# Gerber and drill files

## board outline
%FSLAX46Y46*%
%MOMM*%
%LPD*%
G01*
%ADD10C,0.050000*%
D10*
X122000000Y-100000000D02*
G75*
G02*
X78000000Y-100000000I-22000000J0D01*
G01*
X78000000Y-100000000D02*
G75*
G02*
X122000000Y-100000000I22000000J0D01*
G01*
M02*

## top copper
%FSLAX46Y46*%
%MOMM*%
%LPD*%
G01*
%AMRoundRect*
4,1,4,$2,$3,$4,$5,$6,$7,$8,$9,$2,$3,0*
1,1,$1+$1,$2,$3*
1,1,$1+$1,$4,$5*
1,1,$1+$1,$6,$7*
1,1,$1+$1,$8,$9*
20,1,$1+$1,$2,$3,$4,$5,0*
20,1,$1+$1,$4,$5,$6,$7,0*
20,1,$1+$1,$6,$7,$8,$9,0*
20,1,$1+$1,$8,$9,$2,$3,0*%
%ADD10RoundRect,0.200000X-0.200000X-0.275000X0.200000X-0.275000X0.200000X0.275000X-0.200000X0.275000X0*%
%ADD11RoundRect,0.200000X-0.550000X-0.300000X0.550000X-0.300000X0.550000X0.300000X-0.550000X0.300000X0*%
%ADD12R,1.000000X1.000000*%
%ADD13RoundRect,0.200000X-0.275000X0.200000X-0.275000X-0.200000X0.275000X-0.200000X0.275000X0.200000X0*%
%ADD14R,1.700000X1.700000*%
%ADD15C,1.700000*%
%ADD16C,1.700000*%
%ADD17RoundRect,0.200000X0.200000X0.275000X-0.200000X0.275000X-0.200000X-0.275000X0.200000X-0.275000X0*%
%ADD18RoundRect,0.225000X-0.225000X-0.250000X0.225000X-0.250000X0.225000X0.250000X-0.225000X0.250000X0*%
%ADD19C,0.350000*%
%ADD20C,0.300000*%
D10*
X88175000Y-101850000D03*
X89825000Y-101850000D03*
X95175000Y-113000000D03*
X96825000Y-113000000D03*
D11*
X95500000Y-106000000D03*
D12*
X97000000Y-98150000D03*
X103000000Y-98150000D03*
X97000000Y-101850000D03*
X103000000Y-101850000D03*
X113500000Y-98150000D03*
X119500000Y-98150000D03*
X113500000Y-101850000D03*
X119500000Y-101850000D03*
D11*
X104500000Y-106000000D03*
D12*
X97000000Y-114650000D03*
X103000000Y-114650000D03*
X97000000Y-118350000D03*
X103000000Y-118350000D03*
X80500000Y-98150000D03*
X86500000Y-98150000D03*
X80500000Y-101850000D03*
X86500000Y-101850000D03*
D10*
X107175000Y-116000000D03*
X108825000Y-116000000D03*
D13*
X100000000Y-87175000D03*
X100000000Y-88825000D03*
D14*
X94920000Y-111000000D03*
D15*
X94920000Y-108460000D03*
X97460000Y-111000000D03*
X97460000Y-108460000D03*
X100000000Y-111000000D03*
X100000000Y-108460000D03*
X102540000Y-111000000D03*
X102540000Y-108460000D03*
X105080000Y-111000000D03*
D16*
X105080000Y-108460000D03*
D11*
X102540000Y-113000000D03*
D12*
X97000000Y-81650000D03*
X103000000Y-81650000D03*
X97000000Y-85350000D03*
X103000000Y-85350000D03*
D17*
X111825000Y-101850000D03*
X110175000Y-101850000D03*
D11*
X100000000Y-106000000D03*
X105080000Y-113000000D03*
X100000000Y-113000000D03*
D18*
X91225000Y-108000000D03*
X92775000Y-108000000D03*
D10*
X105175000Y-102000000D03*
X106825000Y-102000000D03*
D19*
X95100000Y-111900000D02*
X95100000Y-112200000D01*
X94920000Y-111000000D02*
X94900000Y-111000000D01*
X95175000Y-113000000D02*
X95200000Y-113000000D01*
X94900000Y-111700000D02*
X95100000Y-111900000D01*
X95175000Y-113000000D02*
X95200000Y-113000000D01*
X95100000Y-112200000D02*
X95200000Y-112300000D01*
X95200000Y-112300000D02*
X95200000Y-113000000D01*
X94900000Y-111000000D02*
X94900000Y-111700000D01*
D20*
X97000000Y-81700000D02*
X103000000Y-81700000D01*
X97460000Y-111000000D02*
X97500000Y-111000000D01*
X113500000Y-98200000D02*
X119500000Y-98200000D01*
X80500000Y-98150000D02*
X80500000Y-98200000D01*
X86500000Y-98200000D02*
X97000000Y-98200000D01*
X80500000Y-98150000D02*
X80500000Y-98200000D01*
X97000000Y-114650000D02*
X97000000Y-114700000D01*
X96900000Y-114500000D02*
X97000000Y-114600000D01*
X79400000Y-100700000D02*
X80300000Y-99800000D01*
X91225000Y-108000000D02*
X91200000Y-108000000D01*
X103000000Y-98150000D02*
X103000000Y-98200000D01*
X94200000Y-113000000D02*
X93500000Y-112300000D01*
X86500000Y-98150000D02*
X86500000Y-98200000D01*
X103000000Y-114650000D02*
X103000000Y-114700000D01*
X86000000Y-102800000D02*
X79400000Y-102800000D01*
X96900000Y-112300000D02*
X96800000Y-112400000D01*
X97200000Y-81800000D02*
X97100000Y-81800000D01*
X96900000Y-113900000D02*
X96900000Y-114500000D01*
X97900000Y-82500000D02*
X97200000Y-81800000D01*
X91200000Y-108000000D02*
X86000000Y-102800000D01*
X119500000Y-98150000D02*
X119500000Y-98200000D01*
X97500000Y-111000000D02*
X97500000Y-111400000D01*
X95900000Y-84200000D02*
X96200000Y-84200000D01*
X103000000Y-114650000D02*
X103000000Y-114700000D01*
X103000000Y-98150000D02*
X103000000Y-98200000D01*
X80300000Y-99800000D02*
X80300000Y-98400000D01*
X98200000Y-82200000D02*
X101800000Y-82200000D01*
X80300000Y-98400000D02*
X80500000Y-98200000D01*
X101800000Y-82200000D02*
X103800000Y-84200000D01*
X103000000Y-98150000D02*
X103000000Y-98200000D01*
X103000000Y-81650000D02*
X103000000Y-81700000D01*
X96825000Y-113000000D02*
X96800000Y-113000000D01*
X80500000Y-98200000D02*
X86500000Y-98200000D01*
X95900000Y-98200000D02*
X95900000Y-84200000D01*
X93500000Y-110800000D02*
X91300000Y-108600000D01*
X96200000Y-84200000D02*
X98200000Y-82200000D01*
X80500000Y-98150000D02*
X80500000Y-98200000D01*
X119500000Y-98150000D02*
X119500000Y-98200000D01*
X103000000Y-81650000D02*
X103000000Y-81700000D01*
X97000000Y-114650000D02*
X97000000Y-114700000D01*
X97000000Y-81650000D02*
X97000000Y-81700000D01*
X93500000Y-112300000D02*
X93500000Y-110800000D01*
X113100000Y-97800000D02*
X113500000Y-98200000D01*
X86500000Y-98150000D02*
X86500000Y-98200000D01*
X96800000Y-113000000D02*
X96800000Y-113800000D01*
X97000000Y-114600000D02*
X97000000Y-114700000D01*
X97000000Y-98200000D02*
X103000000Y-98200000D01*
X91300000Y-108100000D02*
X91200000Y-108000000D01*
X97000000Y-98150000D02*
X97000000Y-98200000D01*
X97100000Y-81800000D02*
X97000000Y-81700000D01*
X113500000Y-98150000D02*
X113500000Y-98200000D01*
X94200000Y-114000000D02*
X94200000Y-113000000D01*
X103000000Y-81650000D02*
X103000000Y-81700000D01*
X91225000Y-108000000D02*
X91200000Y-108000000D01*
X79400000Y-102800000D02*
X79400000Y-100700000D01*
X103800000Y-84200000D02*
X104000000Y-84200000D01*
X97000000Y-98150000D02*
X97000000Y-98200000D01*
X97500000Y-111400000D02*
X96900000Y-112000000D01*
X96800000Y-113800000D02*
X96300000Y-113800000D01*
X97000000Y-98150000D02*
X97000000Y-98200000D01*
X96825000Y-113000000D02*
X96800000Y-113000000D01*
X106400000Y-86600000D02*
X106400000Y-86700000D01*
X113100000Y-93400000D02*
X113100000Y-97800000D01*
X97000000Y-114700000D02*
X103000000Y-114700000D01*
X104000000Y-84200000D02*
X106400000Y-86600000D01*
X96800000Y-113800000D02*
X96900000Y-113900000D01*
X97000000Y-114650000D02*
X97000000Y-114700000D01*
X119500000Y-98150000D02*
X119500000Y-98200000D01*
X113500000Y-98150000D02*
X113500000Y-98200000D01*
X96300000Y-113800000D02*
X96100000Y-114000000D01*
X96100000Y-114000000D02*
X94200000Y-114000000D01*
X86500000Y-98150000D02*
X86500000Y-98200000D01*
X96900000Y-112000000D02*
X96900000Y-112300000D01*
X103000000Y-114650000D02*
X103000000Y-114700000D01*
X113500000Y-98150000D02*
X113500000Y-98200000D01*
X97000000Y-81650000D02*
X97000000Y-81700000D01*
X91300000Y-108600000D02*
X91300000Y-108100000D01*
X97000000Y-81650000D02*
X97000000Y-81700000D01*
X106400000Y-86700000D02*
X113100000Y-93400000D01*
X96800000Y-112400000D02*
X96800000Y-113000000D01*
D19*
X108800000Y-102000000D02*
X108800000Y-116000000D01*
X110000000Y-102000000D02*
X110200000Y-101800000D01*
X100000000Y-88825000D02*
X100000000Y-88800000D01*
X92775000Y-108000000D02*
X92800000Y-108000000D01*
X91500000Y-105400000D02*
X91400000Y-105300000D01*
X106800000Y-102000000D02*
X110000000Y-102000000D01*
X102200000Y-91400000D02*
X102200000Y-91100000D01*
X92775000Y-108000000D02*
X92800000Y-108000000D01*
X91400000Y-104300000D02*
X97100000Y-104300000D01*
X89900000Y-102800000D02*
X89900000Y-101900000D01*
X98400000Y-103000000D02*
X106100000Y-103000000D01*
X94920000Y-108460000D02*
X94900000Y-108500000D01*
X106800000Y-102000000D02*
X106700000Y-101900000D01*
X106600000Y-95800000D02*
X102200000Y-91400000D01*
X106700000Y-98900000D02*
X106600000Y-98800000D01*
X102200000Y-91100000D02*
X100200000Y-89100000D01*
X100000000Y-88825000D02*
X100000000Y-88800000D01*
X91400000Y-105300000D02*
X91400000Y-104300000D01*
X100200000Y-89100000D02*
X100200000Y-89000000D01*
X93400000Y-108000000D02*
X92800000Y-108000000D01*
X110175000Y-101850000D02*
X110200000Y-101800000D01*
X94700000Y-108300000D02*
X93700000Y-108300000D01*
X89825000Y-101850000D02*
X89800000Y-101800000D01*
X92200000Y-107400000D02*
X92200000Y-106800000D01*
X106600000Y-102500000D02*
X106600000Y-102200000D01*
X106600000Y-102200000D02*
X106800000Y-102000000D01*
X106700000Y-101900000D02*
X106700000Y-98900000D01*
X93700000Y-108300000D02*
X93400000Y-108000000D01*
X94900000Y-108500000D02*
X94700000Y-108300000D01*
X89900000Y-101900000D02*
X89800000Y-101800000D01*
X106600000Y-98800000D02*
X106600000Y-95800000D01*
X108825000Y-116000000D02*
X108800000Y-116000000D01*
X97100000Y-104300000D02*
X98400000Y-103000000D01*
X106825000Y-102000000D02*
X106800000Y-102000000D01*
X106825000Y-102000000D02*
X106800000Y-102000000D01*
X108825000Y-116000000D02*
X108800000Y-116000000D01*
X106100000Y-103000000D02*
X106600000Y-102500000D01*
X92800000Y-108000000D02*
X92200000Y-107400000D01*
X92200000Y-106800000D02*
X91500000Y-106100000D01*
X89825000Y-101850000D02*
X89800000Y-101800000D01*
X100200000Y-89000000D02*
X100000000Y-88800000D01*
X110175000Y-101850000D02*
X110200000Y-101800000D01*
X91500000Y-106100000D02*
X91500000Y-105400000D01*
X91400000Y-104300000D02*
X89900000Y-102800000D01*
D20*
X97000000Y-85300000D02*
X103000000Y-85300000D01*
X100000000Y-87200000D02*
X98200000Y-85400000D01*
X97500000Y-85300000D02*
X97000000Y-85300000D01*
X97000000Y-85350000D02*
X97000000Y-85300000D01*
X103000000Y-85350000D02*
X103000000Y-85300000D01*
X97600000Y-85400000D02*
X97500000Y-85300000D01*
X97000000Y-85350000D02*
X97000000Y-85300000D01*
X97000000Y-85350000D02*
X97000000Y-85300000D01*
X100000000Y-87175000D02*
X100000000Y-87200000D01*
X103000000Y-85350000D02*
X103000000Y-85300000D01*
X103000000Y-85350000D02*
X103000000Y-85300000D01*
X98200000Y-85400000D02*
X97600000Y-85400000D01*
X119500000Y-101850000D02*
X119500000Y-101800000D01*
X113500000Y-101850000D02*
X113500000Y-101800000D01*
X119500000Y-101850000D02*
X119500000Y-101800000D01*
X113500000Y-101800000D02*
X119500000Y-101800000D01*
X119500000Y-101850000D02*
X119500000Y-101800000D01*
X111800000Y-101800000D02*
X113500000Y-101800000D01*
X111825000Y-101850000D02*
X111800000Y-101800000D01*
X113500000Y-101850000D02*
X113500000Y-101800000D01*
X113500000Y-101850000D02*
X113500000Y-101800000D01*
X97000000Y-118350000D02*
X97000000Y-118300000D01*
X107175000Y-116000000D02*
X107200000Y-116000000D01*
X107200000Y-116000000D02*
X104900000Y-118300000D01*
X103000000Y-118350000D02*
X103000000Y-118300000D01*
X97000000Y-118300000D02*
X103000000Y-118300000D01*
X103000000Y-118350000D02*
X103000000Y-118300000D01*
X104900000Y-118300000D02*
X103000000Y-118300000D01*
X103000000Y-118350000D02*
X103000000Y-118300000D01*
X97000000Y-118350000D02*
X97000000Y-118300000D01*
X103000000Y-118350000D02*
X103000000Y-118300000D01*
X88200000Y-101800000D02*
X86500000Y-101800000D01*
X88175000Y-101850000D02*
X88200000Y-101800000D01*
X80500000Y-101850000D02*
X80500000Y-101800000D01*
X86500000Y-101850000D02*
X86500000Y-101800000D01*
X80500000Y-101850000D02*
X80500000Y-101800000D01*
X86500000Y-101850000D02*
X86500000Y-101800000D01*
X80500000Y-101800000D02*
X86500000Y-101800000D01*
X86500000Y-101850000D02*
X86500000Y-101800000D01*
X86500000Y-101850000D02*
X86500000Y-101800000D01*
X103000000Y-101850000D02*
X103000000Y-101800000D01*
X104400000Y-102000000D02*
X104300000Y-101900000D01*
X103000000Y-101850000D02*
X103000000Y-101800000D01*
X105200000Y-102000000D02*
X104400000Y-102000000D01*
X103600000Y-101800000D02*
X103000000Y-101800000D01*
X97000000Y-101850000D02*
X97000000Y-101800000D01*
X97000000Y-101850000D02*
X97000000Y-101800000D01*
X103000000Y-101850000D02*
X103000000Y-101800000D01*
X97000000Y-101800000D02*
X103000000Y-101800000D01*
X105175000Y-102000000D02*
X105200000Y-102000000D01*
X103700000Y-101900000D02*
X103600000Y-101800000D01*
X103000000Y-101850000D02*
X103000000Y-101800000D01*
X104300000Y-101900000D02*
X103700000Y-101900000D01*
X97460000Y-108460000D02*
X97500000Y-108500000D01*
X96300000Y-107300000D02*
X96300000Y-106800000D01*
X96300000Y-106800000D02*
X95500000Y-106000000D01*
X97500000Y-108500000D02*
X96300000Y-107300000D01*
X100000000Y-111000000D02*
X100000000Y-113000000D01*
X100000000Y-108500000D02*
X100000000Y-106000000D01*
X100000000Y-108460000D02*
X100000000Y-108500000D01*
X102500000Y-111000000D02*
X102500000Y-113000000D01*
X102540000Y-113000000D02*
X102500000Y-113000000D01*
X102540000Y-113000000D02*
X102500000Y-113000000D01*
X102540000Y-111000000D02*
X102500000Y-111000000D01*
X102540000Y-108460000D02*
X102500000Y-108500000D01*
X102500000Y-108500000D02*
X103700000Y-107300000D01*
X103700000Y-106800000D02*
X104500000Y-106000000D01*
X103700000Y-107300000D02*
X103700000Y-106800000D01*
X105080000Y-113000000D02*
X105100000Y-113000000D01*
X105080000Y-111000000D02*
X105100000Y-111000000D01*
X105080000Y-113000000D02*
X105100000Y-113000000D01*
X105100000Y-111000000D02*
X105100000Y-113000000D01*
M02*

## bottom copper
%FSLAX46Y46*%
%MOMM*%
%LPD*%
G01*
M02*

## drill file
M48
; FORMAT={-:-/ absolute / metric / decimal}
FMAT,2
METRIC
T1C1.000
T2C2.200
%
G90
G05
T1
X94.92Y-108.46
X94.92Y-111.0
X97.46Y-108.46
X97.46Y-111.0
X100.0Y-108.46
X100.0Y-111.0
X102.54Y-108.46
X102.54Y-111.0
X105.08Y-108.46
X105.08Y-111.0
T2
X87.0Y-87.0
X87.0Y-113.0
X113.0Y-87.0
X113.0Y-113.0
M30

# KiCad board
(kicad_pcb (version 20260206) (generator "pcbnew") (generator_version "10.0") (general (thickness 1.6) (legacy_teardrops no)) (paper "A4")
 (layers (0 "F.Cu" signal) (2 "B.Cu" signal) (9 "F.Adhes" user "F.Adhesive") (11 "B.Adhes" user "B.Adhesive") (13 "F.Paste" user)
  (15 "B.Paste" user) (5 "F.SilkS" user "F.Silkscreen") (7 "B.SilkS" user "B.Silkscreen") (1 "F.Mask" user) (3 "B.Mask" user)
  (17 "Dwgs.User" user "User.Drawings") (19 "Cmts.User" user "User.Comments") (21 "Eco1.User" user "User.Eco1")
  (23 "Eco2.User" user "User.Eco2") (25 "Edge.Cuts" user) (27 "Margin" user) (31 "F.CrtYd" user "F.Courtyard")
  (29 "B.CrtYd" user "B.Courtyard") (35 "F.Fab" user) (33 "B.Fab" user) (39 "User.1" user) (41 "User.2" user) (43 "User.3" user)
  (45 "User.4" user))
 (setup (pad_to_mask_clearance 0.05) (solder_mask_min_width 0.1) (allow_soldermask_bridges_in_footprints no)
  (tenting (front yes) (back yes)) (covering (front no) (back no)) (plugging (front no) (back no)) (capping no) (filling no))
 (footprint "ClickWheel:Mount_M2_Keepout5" (layer "F.Cu") (at 87 113)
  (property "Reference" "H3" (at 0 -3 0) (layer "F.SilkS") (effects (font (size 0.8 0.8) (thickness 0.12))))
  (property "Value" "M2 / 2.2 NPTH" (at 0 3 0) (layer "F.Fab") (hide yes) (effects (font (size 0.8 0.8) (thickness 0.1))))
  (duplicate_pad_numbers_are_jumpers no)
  (pad "" np_thru_hole circle (at 0 0) (size 2.2 2.2) (drill 2.2) (layers "*.Cu" "*.Mask")))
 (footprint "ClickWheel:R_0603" (layer "F.Cu") (at 89 101.85)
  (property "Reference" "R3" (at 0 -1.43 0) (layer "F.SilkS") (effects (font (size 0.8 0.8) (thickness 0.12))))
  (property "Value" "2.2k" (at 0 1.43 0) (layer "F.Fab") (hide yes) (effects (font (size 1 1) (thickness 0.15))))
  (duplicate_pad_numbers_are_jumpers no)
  (pad "1" smd roundrect (at -0.825 0) (size 0.8 0.95) (layers "F.Cu" "F.Mask" "F.Paste") (roundrect_rratio 0.25) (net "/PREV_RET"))
  (pad "2" smd roundrect (at 0.825 0) (size 0.8 0.95) (layers "F.Cu" "F.Mask" "F.Paste") (roundrect_rratio 0.25) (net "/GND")))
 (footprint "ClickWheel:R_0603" (layer "F.Cu") (at 96 113)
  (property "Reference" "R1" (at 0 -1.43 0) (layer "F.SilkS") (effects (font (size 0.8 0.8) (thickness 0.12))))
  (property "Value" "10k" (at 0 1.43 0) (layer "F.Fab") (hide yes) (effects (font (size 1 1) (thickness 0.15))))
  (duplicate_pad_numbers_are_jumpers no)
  (pad "1" smd roundrect (at -0.825 0) (size 0.8 0.95) (layers "F.Cu" "F.Mask" "F.Paste") (roundrect_rratio 0.25) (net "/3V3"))
  (pad "2" smd roundrect (at 0.825 0) (size 0.8 0.95) (layers "F.Cu" "F.Mask" "F.Paste") (roundrect_rratio 0.25) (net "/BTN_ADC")))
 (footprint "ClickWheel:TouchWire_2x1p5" (layer "F.Cu") (at 95.5 106)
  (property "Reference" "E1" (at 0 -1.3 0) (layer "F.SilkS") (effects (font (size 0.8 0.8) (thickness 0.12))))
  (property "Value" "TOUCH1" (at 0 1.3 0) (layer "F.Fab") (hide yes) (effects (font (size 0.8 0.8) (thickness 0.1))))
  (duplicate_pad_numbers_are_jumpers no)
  (pad "1" smd roundrect (at 0 0) (size 1.5 1) (layers "F.Cu" "F.Mask") (roundrect_rratio 0.2) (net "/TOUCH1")))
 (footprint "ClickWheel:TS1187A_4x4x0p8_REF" (layer "F.Cu") (at 100 100)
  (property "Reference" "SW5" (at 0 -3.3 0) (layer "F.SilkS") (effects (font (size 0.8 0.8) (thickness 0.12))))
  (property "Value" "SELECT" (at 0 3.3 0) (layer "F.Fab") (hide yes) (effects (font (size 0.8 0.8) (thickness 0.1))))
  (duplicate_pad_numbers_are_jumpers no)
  (pad "1" smd rect (at -3 -1.85) (size 1 1) (layers "F.Cu" "F.Mask" "F.Paste") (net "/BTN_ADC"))
  (pad "1" smd rect (at 3 -1.85) (size 1 1) (layers "F.Cu" "F.Mask" "F.Paste") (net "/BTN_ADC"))
  (pad "2" smd rect (at -3 1.85) (size 1 1) (layers "F.Cu" "F.Mask" "F.Paste") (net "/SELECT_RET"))
  (pad "2" smd rect (at 3 1.85) (size 1 1) (layers "F.Cu" "F.Mask" "F.Paste") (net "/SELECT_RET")))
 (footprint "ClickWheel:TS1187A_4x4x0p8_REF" (layer "F.Cu") (at 116.5 100)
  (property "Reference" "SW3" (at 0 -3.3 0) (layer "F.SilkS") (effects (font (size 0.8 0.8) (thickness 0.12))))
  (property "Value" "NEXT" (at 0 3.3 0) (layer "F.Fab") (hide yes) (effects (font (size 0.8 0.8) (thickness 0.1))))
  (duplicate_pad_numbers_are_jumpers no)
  (pad "1" smd rect (at -3 -1.85) (size 1 1) (layers "F.Cu" "F.Mask" "F.Paste") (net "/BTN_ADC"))
  (pad "1" smd rect (at 3 -1.85) (size 1 1) (layers "F.Cu" "F.Mask" "F.Paste") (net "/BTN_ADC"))
  (pad "2" smd rect (at -3 1.85) (size 1 1) (layers "F.Cu" "F.Mask" "F.Paste") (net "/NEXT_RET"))
  (pad "2" smd rect (at 3 1.85) (size 1 1) (layers "F.Cu" "F.Mask" "F.Paste") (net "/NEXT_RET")))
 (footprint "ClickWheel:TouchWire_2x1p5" (layer "F.Cu") (at 104.5 106)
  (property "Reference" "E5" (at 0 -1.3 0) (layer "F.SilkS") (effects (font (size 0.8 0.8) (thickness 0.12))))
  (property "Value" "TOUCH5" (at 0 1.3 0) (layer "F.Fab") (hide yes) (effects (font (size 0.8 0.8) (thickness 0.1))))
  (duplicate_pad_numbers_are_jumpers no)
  (pad "1" smd roundrect (at 0 0) (size 1.5 1) (layers "F.Cu" "F.Mask") (roundrect_rratio 0.2) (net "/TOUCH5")))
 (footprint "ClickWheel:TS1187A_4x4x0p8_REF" (layer "F.Cu") (at 100 116.5)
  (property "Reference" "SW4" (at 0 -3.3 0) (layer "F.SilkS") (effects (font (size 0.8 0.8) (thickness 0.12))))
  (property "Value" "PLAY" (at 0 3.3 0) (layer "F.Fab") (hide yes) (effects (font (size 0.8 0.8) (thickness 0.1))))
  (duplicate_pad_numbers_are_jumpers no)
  (pad "1" smd rect (at -3 -1.85) (size 1 1) (layers "F.Cu" "F.Mask" "F.Paste") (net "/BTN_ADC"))
  (pad "1" smd rect (at 3 -1.85) (size 1 1) (layers "F.Cu" "F.Mask" "F.Paste") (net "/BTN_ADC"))
  (pad "2" smd rect (at -3 1.85) (size 1 1) (layers "F.Cu" "F.Mask" "F.Paste") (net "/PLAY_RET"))
  (pad "2" smd rect (at 3 1.85) (size 1 1) (layers "F.Cu" "F.Mask" "F.Paste") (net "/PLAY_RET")))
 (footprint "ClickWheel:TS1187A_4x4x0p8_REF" (layer "F.Cu") (at 83.5 100)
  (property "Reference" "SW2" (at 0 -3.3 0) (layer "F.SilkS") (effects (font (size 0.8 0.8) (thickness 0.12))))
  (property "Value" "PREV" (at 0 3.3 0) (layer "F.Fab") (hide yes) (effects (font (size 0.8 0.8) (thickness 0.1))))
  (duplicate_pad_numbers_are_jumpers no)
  (pad "1" smd rect (at -3 -1.85) (size 1 1) (layers "F.Cu" "F.Mask" "F.Paste") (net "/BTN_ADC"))
  (pad "1" smd rect (at 3 -1.85) (size 1 1) (layers "F.Cu" "F.Mask" "F.Paste") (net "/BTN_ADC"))
  (pad "2" smd rect (at -3 1.85) (size 1 1) (layers "F.Cu" "F.Mask" "F.Paste") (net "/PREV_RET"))
  (pad "2" smd rect (at 3 1.85) (size 1 1) (layers "F.Cu" "F.Mask" "F.Paste") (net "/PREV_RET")))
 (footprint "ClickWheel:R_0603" (layer "F.Cu") (at 108 116)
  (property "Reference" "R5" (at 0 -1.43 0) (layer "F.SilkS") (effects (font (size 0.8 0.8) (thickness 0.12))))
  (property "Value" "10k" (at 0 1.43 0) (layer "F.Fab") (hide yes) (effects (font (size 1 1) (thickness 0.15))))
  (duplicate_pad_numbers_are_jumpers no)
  (pad "1" smd roundrect (at -0.825 0) (size 0.8 0.95) (layers "F.Cu" "F.Mask" "F.Paste") (roundrect_rratio 0.25) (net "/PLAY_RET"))
  (pad "2" smd roundrect (at 0.825 0) (size 0.8 0.95) (layers "F.Cu" "F.Mask" "F.Paste") (roundrect_rratio 0.25) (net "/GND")))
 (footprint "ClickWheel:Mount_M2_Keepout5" (layer "F.Cu") (at 113 113)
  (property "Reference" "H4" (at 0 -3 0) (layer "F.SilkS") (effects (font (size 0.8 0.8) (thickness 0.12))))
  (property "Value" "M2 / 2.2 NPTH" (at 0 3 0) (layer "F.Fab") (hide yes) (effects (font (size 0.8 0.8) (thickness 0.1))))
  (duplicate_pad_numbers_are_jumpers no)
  (pad "" np_thru_hole circle (at 0 0) (size 2.2 2.2) (drill 2.2) (layers "*.Cu" "*.Mask")))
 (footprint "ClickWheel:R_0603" (layer "F.Cu") (at 100 88 -90)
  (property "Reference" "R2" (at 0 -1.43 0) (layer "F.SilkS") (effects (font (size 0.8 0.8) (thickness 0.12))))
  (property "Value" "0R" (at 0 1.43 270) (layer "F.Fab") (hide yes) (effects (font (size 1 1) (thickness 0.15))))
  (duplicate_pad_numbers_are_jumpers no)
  (pad "1" smd roundrect (at -0.825 0 270) (size 0.8 0.95) (layers "F.Cu" "F.Mask" "F.Paste") (roundrect_rratio 0.25) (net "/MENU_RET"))
  (pad "2" smd roundrect (at 0.825 0 270) (size 0.8 0.95) (layers "F.Cu" "F.Mask" "F.Paste") (roundrect_rratio 0.25) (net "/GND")))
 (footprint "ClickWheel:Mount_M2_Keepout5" (layer "F.Cu") (at 113 87)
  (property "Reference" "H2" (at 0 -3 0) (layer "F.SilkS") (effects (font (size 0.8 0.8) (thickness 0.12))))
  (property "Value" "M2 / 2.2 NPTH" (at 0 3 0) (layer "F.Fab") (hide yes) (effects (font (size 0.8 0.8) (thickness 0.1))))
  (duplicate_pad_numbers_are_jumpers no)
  (pad "" np_thru_hole circle (at 0 0) (size 2.2 2.2) (drill 2.2) (layers "*.Cu" "*.Mask")))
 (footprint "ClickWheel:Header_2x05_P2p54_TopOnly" (layer "F.Cu") (at 94.92 111 90)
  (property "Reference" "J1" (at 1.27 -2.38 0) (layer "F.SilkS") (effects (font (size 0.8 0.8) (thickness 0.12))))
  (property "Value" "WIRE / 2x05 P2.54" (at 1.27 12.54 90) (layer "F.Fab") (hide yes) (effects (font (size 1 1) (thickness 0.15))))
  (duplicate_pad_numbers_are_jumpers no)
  (pad "1" thru_hole rect (at 0 0 90) (size 1.7 1.7) (drill 1) (layers "*.Mask" "F.Cu") (remove_unused_layers yes) (keep_end_layers no)
   (zone_layer_connections) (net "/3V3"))
  (pad "2" thru_hole circle (at 2.54 0 90) (size 1.7 1.7) (drill 1) (layers "*.Mask" "F.Cu") (remove_unused_layers yes) (keep_end_layers no)
   (zone_layer_connections) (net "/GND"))
  (pad "3" thru_hole circle (at 0 2.54 90) (size 1.7 1.7) (drill 1) (layers "*.Mask" "F.Cu") (remove_unused_layers yes) (keep_end_layers no)
   (zone_layer_connections) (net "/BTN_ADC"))
  (pad "4" thru_hole circle (at 2.54 2.54 90) (size 1.7 1.7) (drill 1) (layers "*.Mask" "F.Cu") (remove_unused_layers yes)
   (keep_end_layers no) (zone_layer_connections) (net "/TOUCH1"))
  (pad "5" thru_hole circle (at 0 5.08 90) (size 1.7 1.7) (drill 1) (layers "*.Mask" "F.Cu") (remove_unused_layers yes) (keep_end_layers no)
   (zone_layer_connections) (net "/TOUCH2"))
  (pad "6" thru_hole circle (at 2.54 5.08 90) (size 1.7 1.7) (drill 1) (layers "*.Mask" "F.Cu") (remove_unused_layers yes)
   (keep_end_layers no) (zone_layer_connections) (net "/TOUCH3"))
  (pad "7" thru_hole circle (at 0 7.62 90) (size 1.7 1.7) (drill 1) (layers "*.Mask" "F.Cu") (remove_unused_layers yes) (keep_end_layers no)
   (zone_layer_connections) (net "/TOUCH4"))
  (pad "8" thru_hole circle (at 2.54 7.62 90) (size 1.7 1.7) (drill 1) (layers "*.Mask" "F.Cu") (remove_unused_layers yes)
   (keep_end_layers no) (zone_layer_connections) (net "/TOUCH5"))
  (pad "9" thru_hole circle (at 0 10.16 90) (size 1.7 1.7) (drill 1) (layers "*.Mask" "F.Cu") (remove_unused_layers yes)
   (keep_end_layers no) (zone_layer_connections) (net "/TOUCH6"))
  (pad "10" smd circle (at 2.54 10.16 90) (size 1.7 1.7) (layers "F.Cu" "F.Mask"))
  (pad "10" thru_hole circle (at 2.54 10.16 90) (size 1.7 1.7) (drill 1) (layers "*.Mask" "F.Cu") (remove_unused_layers yes)
   (keep_end_layers no) (zone_layer_connections)))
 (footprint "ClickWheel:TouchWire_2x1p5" (layer "F.Cu") (at 102.54 113)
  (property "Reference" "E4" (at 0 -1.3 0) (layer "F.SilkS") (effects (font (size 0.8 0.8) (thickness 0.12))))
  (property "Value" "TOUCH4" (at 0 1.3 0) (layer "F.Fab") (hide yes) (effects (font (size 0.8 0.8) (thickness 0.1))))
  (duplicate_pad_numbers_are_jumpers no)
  (pad "1" smd roundrect (at 0 0) (size 1.5 1) (layers "F.Cu" "F.Mask") (roundrect_rratio 0.2) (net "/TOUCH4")))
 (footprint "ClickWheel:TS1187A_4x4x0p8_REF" (layer "F.Cu") (at 100 83.5)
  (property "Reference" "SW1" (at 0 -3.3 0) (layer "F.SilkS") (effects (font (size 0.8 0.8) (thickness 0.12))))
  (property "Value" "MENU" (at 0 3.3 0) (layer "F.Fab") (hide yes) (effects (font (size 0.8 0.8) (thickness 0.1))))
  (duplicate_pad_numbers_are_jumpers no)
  (pad "1" smd rect (at -3 -1.85) (size 1 1) (layers "F.Cu" "F.Mask" "F.Paste") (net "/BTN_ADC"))
  (pad "1" smd rect (at 3 -1.85) (size 1 1) (layers "F.Cu" "F.Mask" "F.Paste") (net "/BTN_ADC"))
  (pad "2" smd rect (at -3 1.85) (size 1 1) (layers "F.Cu" "F.Mask" "F.Paste") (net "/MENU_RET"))
  (pad "2" smd rect (at 3 1.85) (size 1 1) (layers "F.Cu" "F.Mask" "F.Paste") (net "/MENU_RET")))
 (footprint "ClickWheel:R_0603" (layer "F.Cu") (at 111 101.85 180)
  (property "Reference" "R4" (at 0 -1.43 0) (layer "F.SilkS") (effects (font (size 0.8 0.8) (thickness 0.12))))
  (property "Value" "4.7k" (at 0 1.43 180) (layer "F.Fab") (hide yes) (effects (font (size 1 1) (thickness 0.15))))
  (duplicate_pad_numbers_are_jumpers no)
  (pad "1" smd roundrect (at -0.825 0 180) (size 0.8 0.95) (layers "F.Cu" "F.Mask" "F.Paste") (roundrect_rratio 0.25) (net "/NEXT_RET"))
  (pad "2" smd roundrect (at 0.825 0 180) (size 0.8 0.95) (layers "F.Cu" "F.Mask" "F.Paste") (roundrect_rratio 0.25) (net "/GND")))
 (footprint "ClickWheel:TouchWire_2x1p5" (layer "F.Cu") (at 100 106)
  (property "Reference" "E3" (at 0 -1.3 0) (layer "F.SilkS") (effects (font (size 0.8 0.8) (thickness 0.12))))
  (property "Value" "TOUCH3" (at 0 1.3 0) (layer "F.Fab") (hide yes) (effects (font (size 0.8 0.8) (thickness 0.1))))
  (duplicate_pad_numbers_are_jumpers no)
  (pad "1" smd roundrect (at 0 0) (size 1.5 1) (layers "F.Cu" "F.Mask") (roundrect_rratio 0.2) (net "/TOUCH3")))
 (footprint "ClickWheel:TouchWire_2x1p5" (layer "F.Cu") (at 105.08 113)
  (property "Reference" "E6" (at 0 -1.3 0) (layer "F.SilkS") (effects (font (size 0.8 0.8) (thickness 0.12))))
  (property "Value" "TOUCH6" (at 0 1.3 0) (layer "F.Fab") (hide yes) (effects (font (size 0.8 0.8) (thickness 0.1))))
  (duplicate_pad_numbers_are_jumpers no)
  (pad "1" smd roundrect (at 0 0) (size 1.5 1) (layers "F.Cu" "F.Mask") (roundrect_rratio 0.2) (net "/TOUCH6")))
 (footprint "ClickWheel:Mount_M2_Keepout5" (layer "F.Cu") (at 87 87)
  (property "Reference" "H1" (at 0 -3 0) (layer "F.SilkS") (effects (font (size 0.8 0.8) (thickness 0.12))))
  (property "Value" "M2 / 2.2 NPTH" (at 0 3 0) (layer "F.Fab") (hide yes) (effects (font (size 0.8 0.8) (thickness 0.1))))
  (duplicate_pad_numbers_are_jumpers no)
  (pad "" np_thru_hole circle (at 0 0) (size 2.2 2.2) (drill 2.2) (layers "*.Cu" "*.Mask")))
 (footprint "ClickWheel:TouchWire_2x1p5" (layer "F.Cu") (at 100 113)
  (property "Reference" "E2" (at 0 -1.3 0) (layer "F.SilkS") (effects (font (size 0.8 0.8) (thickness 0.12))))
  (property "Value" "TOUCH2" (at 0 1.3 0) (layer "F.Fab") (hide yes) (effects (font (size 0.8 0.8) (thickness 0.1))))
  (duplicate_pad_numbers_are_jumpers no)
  (pad "1" smd roundrect (at 0 0) (size 1.5 1) (layers "F.Cu" "F.Mask") (roundrect_rratio 0.2) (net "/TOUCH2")))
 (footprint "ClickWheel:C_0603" (layer "F.Cu") (at 92 108)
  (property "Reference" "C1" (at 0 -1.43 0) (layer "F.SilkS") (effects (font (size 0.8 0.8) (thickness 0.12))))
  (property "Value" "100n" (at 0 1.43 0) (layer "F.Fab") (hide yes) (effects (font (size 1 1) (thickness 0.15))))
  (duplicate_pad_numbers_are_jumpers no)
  (pad "1" smd roundrect (at -0.775 0) (size 0.9 0.95) (layers "F.Cu" "F.Mask" "F.Paste") (roundrect_rratio 0.25) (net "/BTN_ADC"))
  (pad "2" smd roundrect (at 0.775 0) (size 0.9 0.95) (layers "F.Cu" "F.Mask" "F.Paste") (roundrect_rratio 0.25) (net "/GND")))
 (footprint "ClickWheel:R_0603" (layer "F.Cu") (at 106 102)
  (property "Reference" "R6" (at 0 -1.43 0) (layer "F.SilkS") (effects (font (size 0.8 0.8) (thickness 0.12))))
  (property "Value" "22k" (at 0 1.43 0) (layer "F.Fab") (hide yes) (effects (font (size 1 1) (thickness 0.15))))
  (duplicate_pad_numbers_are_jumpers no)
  (pad "1" smd roundrect (at -0.825 0) (size 0.8 0.95) (layers "F.Cu" "F.Mask" "F.Paste") (roundrect_rratio 0.25) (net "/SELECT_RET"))
  (pad "2" smd roundrect (at 0.825 0) (size 0.8 0.95) (layers "F.Cu" "F.Mask" "F.Paste") (roundrect_rratio 0.25) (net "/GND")))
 (gr_circle (center 100 100) (end 122 100) (stroke (width 0.05) (type default)) (fill no) (layer "Edge.Cuts"))
 (segment (start 95.1 111.9) (end 95.1 112.2) (width 0.35) (layer "F.Cu") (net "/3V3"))
 (segment (start 94.92 111) (end 94.9 111) (width 0.35) (layer "F.Cu") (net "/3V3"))
 (segment (start 95.175 113) (end 95.2 113) (width 0.35) (layer "F.Cu") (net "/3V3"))
 (segment (start 94.9 111.7) (end 95.1 111.9) (width 0.35) (layer "F.Cu") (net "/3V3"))
 (segment (start 95.175 113) (end 95.2 113) (width 0.35) (layer "F.Cu") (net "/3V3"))
 (segment (start 95.1 112.2) (end 95.2 112.3) (width 0.35) (layer "F.Cu") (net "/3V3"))
 (segment (start 95.2 112.3) (end 95.2 113) (width 0.35) (layer "F.Cu") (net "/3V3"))
 (segment (start 94.9 111) (end 94.9 111.7) (width 0.35) (layer "F.Cu") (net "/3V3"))
 (segment (start 97 81.7) (end 103 81.7) (width 0.3) (layer "F.Cu") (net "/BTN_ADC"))
 (segment (start 97.46 111) (end 97.5 111) (width 0.3) (layer "F.Cu") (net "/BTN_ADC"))
 (segment (start 113.5 98.2) (end 119.5 98.2) (width 0.3) (layer "F.Cu") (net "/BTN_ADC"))
 (segment (start 80.5 98.15) (end 80.5 98.2) (width 0.3) (layer "F.Cu") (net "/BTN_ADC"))
 (segment (start 86.5 98.2) (end 97 98.2) (width 0.3) (layer "F.Cu") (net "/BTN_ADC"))
 (segment (start 80.5 98.15) (end 80.5 98.2) (width 0.3) (layer "F.Cu") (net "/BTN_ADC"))
 (segment (start 97 114.65) (end 97 114.7) (width 0.3) (layer "F.Cu") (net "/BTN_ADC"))
 (segment (start 96.9 114.5) (end 97 114.6) (width 0.3) (layer "F.Cu") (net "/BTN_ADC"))
 (segment (start 79.4 100.7) (end 80.3 99.8) (width 0.3) (layer "F.Cu") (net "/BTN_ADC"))
 (segment (start 91.225 108) (end 91.2 108) (width 0.3) (layer "F.Cu") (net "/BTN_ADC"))
 (segment (start 103 98.15) (end 103 98.2) (width 0.3) (layer "F.Cu") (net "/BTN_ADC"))
 (segment (start 94.2 113) (end 93.5 112.3) (width 0.3) (layer "F.Cu") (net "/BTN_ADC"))
 (segment (start 86.5 98.15) (end 86.5 98.2) (width 0.3) (layer "F.Cu") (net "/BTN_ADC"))
 (segment (start 103 114.65) (end 103 114.7) (width 0.3) (layer "F.Cu") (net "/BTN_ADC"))
 (segment (start 86 102.8) (end 79.4 102.8) (width 0.3) (layer "F.Cu") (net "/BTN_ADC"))
 (segment (start 96.9 112.3) (end 96.8 112.4) (width 0.3) (layer "F.Cu") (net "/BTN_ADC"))
 (segment (start 97.2 81.8) (end 97.1 81.8) (width 0.3) (layer "F.Cu") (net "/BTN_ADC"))
 (segment (start 96.9 113.9) (end 96.9 114.5) (width 0.3) (layer "F.Cu") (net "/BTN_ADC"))
 (segment (start 97.9 82.5) (end 97.2 81.8) (width 0.3) (layer "F.Cu") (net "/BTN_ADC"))
 (segment (start 91.2 108) (end 86 102.8) (width 0.3) (layer "F.Cu") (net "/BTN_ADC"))
 (segment (start 119.5 98.15) (end 119.5 98.2) (width 0.3) (layer "F.Cu") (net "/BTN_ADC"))
 (segment (start 97.5 111) (end 97.5 111.4) (width 0.3) (layer "F.Cu") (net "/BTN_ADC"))
 (segment (start 95.9 84.2) (end 96.2 84.2) (width 0.3) (layer "F.Cu") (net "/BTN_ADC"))
 (segment (start 103 114.65) (end 103 114.7) (width 0.3) (layer "F.Cu") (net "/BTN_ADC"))
 (segment (start 103 98.15) (end 103 98.2) (width 0.3) (layer "F.Cu") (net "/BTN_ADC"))
 (segment (start 80.3 99.8) (end 80.3 98.4) (width 0.3) (layer "F.Cu") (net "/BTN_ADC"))
 (segment (start 98.2 82.2) (end 101.8 82.2) (width 0.3) (layer "F.Cu") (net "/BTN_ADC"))
 (segment (start 80.3 98.4) (end 80.5 98.2) (width 0.3) (layer "F.Cu") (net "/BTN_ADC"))
 (segment (start 101.8 82.2) (end 103.8 84.2) (width 0.3) (layer "F.Cu") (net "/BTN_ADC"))
 (segment (start 103 98.15) (end 103 98.2) (width 0.3) (layer "F.Cu") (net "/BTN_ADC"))
 (segment (start 103 81.65) (end 103 81.7) (width 0.3) (layer "F.Cu") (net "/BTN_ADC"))
 (segment (start 96.825 113) (end 96.8 113) (width 0.3) (layer "F.Cu") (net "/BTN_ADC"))
 (segment (start 80.5 98.2) (end 86.5 98.2) (width 0.3) (layer "F.Cu") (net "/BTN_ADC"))
 (segment (start 95.9 98.2) (end 95.9 84.2) (width 0.3) (layer "F.Cu") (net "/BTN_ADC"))
 (segment (start 93.5 110.8) (end 91.3 108.6) (width 0.3) (layer "F.Cu") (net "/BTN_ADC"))
 (segment (start 96.2 84.2) (end 98.2 82.2) (width 0.3) (layer "F.Cu") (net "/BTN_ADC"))
 (segment (start 80.5 98.15) (end 80.5 98.2) (width 0.3) (layer "F.Cu") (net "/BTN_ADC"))
 (segment (start 119.5 98.15) (end 119.5 98.2) (width 0.3) (layer "F.Cu") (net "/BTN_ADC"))
 (segment (start 103 81.65) (end 103 81.7) (width 0.3) (layer "F.Cu") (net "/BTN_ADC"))
 (segment (start 97 114.65) (end 97 114.7) (width 0.3) (layer "F.Cu") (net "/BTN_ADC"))
 (segment (start 97 81.65) (end 97 81.7) (width 0.3) (layer "F.Cu") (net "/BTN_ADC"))
 (segment (start 93.5 112.3) (end 93.5 110.8) (width 0.3) (layer "F.Cu") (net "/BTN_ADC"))
 (segment (start 113.1 97.8) (end 113.5 98.2) (width 0.3) (layer "F.Cu") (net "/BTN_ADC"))
 (segment (start 86.5 98.15) (end 86.5 98.2) (width 0.3) (layer "F.Cu") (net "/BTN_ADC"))
 (segment (start 96.8 113) (end 96.8 113.8) (width 0.3) (layer "F.Cu") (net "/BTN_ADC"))
 (segment (start 97 114.6) (end 97 114.7) (width 0.3) (layer "F.Cu") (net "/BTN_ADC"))
 (segment (start 97 98.2) (end 103 98.2) (width 0.3) (layer "F.Cu") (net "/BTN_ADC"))
 (segment (start 91.3 108.1) (end 91.2 108) (width 0.3) (layer "F.Cu") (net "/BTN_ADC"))
 (segment (start 97 98.15) (end 97 98.2) (width 0.3) (layer "F.Cu") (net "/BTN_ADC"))
 (segment (start 97.1 81.8) (end 97 81.7) (width 0.3) (layer "F.Cu") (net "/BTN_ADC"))
 (segment (start 113.5 98.15) (end 113.5 98.2) (width 0.3) (layer "F.Cu") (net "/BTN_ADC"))
 (segment (start 94.2 114) (end 94.2 113) (width 0.3) (layer "F.Cu") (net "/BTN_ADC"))
 (segment (start 103 81.65) (end 103 81.7) (width 0.3) (layer "F.Cu") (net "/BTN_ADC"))
 (segment (start 91.225 108) (end 91.2 108) (width 0.3) (layer "F.Cu") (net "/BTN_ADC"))
 (segment (start 79.4 102.8) (end 79.4 100.7) (width 0.3) (layer "F.Cu") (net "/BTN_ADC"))
 (segment (start 103.8 84.2) (end 104 84.2) (width 0.3) (layer "F.Cu") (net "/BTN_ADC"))
 (segment (start 97 98.15) (end 97 98.2) (width 0.3) (layer "F.Cu") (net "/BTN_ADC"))
 (segment (start 97.5 111.4) (end 96.9 112) (width 0.3) (layer "F.Cu") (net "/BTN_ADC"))
 (segment (start 96.8 113.8) (end 96.3 113.8) (width 0.3) (layer "F.Cu") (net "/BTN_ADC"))
 (segment (start 97 98.15) (end 97 98.2) (width 0.3) (layer "F.Cu") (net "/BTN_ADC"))
 (segment (start 96.825 113) (end 96.8 113) (width 0.3) (layer "F.Cu") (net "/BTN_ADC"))
 (segment (start 106.4 86.6) (end 106.4 86.7) (width 0.3) (layer "F.Cu") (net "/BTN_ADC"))
 (segment (start 113.1 93.4) (end 113.1 97.8) (width 0.3) (layer "F.Cu") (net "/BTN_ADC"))
 (segment (start 97 114.7) (end 103 114.7) (width 0.3) (layer "F.Cu") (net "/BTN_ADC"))
 (segment (start 104 84.2) (end 106.4 86.6) (width 0.3) (layer "F.Cu") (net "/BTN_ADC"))
 (segment (start 96.8 113.8) (end 96.9 113.9) (width 0.3) (layer "F.Cu") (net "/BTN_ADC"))
 (segment (start 97 114.65) (end 97 114.7) (width 0.3) (layer "F.Cu") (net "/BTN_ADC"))
 (segment (start 119.5 98.15) (end 119.5 98.2) (width 0.3) (layer "F.Cu") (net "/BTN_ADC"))
 (segment (start 113.5 98.15) (end 113.5 98.2) (width 0.3) (layer "F.Cu") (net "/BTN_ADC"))
 (segment (start 96.3 113.8) (end 96.1 114) (width 0.3) (layer "F.Cu") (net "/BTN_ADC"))
 (segment (start 96.1 114) (end 94.2 114) (width 0.3) (layer "F.Cu") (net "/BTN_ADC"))
 (segment (start 86.5 98.15) (end 86.5 98.2) (width 0.3) (layer "F.Cu") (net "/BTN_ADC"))
 (segment (start 96.9 112) (end 96.9 112.3) (width 0.3) (layer "F.Cu") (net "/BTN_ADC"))
 (segment (start 103 114.65) (end 103 114.7) (width 0.3) (layer "F.Cu") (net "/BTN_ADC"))
 (segment (start 113.5 98.15) (end 113.5 98.2) (width 0.3) (layer "F.Cu") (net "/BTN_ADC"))
 (segment (start 97 81.65) (end 97 81.7) (width 0.3) (layer "F.Cu") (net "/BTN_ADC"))
 (segment (start 91.3 108.6) (end 91.3 108.1) (width 0.3) (layer "F.Cu") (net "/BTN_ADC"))
 (segment (start 97 81.65) (end 97 81.7) (width 0.3) (layer "F.Cu") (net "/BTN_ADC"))
 (segment (start 106.4 86.7) (end 113.1 93.4) (width 0.3) (layer "F.Cu") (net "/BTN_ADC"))
 (segment (start 96.8 112.4) (end 96.8 113) (width 0.3) (layer "F.Cu") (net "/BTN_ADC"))
 (segment (start 108.8 102) (end 108.8 116) (width 0.35) (layer "F.Cu") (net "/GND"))
 (segment (start 110 102) (end 110.2 101.8) (width 0.35) (layer "F.Cu") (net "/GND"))
 (segment (start 100 88.825) (end 100 88.8) (width 0.35) (layer "F.Cu") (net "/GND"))
 (segment (start 92.775 108) (end 92.8 108) (width 0.35) (layer "F.Cu") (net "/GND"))
 (segment (start 91.5 105.4) (end 91.4 105.3) (width 0.35) (layer "F.Cu") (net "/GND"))
 (segment (start 106.8 102) (end 110 102) (width 0.35) (layer "F.Cu") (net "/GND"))
 (segment (start 102.2 91.4) (end 102.2 91.1) (width 0.35) (layer "F.Cu") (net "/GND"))
 (segment (start 92.775 108) (end 92.8 108) (width 0.35) (layer "F.Cu") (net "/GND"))
 (segment (start 91.4 104.3) (end 97.1 104.3) (width 0.35) (layer "F.Cu") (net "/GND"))
 (segment (start 89.9 102.8) (end 89.9 101.9) (width 0.35) (layer "F.Cu") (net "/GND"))
 (segment (start 98.4 103) (end 106.1 103) (width 0.35) (layer "F.Cu") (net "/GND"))
 (segment (start 94.92 108.46) (end 94.9 108.5) (width 0.35) (layer "F.Cu") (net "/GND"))
 (segment (start 106.8 102) (end 106.7 101.9) (width 0.35) (layer "F.Cu") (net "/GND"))
 (segment (start 106.6 95.8) (end 102.2 91.4) (width 0.35) (layer "F.Cu") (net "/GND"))
 (segment (start 106.7 98.9) (end 106.6 98.8) (width 0.35) (layer "F.Cu") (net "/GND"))
 (segment (start 102.2 91.1) (end 100.2 89.1) (width 0.35) (layer "F.Cu") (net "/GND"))
 (segment (start 100 88.825) (end 100 88.8) (width 0.35) (layer "F.Cu") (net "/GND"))
 (segment (start 91.4 105.3) (end 91.4 104.3) (width 0.35) (layer "F.Cu") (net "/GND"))
 (segment (start 100.2 89.1) (end 100.2 89) (width 0.35) (layer "F.Cu") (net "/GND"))
 (segment (start 93.4 108) (end 92.8 108) (width 0.35) (layer "F.Cu") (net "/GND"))
 (segment (start 110.175 101.85) (end 110.2 101.8) (width 0.35) (layer "F.Cu") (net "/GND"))
 (segment (start 94.7 108.3) (end 93.7 108.3) (width 0.35) (layer "F.Cu") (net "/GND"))
 (segment (start 89.825 101.85) (end 89.8 101.8) (width 0.35) (layer "F.Cu") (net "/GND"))
 (segment (start 92.2 107.4) (end 92.2 106.8) (width 0.35) (layer "F.Cu") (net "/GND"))
 (segment (start 106.6 102.5) (end 106.6 102.2) (width 0.35) (layer "F.Cu") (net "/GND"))
 (segment (start 106.6 102.2) (end 106.8 102) (width 0.35) (layer "F.Cu") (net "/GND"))
 (segment (start 106.7 101.9) (end 106.7 98.9) (width 0.35) (layer "F.Cu") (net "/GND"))
 (segment (start 93.7 108.3) (end 93.4 108) (width 0.35) (layer "F.Cu") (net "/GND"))
 (segment (start 94.9 108.5) (end 94.7 108.3) (width 0.35) (layer "F.Cu") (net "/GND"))
 (segment (start 89.9 101.9) (end 89.8 101.8) (width 0.35) (layer "F.Cu") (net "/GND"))
 (segment (start 106.6 98.8) (end 106.6 95.8) (width 0.35) (layer "F.Cu") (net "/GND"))
 (segment (start 108.825 116) (end 108.8 116) (width 0.35) (layer "F.Cu") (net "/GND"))
 (segment (start 97.1 104.3) (end 98.4 103) (width 0.35) (layer "F.Cu") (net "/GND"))
 (segment (start 106.825 102) (end 106.8 102) (width 0.35) (layer "F.Cu") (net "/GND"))
 (segment (start 106.825 102) (end 106.8 102) (width 0.35) (layer "F.Cu") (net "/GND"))
 (segment (start 108.825 116) (end 108.8 116) (width 0.35) (layer "F.Cu") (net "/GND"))
 (segment (start 106.1 103) (end 106.6 102.5) (width 0.35) (layer "F.Cu") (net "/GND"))
 (segment (start 92.8 108) (end 92.2 107.4) (width 0.35) (layer "F.Cu") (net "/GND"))
 (segment (start 92.2 106.8) (end 91.5 106.1) (width 0.35) (layer "F.Cu") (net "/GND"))
 (segment (start 89.825 101.85) (end 89.8 101.8) (width 0.35) (layer "F.Cu") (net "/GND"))
 (segment (start 100.2 89) (end 100 88.8) (width 0.35) (layer "F.Cu") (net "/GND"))
 (segment (start 110.175 101.85) (end 110.2 101.8) (width 0.35) (layer "F.Cu") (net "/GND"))
 (segment (start 91.5 106.1) (end 91.5 105.4) (width 0.35) (layer "F.Cu") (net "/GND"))
 (segment (start 91.4 104.3) (end 89.9 102.8) (width 0.35) (layer "F.Cu") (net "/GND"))
 (segment (start 97 85.3) (end 103 85.3) (width 0.3) (layer "F.Cu") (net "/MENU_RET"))
 (segment (start 100 87.2) (end 98.2 85.4) (width 0.3) (layer "F.Cu") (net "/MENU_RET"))
 (segment (start 97.5 85.3) (end 97 85.3) (width 0.3) (layer "F.Cu") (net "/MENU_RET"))
 (segment (start 97 85.35) (end 97 85.3) (width 0.3) (layer "F.Cu") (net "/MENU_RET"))
 (segment (start 103 85.35) (end 103 85.3) (width 0.3) (layer "F.Cu") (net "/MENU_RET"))
 (segment (start 97.6 85.4) (end 97.5 85.3) (width 0.3) (layer "F.Cu") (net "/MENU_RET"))
 (segment (start 97 85.35) (end 97 85.3) (width 0.3) (layer "F.Cu") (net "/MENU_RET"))
 (segment (start 97 85.35) (end 97 85.3) (width 0.3) (layer "F.Cu") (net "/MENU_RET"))
 (segment (start 100 87.175) (end 100 87.2) (width 0.3) (layer "F.Cu") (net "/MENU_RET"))
 (segment (start 103 85.35) (end 103 85.3) (width 0.3) (layer "F.Cu") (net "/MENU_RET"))
 (segment (start 103 85.35) (end 103 85.3) (width 0.3) (layer "F.Cu") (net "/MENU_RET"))
 (segment (start 98.2 85.4) (end 97.6 85.4) (width 0.3) (layer "F.Cu") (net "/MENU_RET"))
 (segment (start 119.5 101.85) (end 119.5 101.8) (width 0.3) (layer "F.Cu") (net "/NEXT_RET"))
 (segment (start 113.5 101.85) (end 113.5 101.8) (width 0.3) (layer "F.Cu") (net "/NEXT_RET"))
 (segment (start 119.5 101.85) (end 119.5 101.8) (width 0.3) (layer "F.Cu") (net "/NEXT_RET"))
 (segment (start 113.5 101.8) (end 119.5 101.8) (width 0.3) (layer "F.Cu") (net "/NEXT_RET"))
 (segment (start 119.5 101.85) (end 119.5 101.8) (width 0.3) (layer "F.Cu") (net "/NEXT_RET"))
 (segment (start 111.8 101.8) (end 113.5 101.8) (width 0.3) (layer "F.Cu") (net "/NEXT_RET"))
 (segment (start 111.825 101.85) (end 111.8 101.8) (width 0.3) (layer "F.Cu") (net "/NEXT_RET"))
 (segment (start 113.5 101.85) (end 113.5 101.8) (width 0.3) (layer "F.Cu") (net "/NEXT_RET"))
 (segment (start 113.5 101.85) (end 113.5 101.8) (width 0.3) (layer "F.Cu") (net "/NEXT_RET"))
 (segment (start 97 118.35) (end 97 118.3) (width 0.3) (layer "F.Cu") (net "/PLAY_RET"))
 (segment (start 107.175 116) (end 107.2 116) (width 0.3) (layer "F.Cu") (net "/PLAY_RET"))
 (segment (start 107.2 116) (end 104.9 118.3) (width 0.3) (layer "F.Cu") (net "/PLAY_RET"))
 (segment (start 103 118.35) (end 103 118.3) (width 0.3) (layer "F.Cu") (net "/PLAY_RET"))
 (segment (start 97 118.3) (end 103 118.3) (width 0.3) (layer "F.Cu") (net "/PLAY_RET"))
 (segment (start 103 118.35) (end 103 118.3) (width 0.3) (layer "F.Cu") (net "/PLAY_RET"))
 (segment (start 104.9 118.3) (end 103 118.3) (width 0.3) (layer "F.Cu") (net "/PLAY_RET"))
 (segment (start 103 118.35) (end 103 118.3) (width 0.3) (layer "F.Cu") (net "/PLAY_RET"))
 (segment (start 97 118.35) (end 97 118.3) (width 0.3) (layer "F.Cu") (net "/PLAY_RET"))
 (segment (start 103 118.35) (end 103 118.3) (width 0.3) (layer "F.Cu") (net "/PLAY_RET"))
 (segment (start 88.2 101.8) (end 86.5 101.8) (width 0.3) (layer "F.Cu") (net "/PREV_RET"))
 (segment (start 88.175 101.85) (end 88.2 101.8) (width 0.3) (layer "F.Cu") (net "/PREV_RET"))
 (segment (start 80.5 101.85) (end 80.5 101.8) (width 0.3) (layer "F.Cu") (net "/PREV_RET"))
 (segment (start 86.5 101.85) (end 86.5 101.8) (width 0.3) (layer "F.Cu") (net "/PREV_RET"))
 (segment (start 80.5 101.85) (end 80.5 101.8) (width 0.3) (layer "F.Cu") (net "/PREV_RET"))
 (segment (start 86.5 101.85) (end 86.5 101.8) (width 0.3) (layer "F.Cu") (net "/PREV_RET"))
 (segment (start 80.5 101.8) (end 86.5 101.8) (width 0.3) (layer "F.Cu") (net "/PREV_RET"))
 (segment (start 86.5 101.85) (end 86.5 101.8) (width 0.3) (layer "F.Cu") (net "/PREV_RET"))
 (segment (start 86.5 101.85) (end 86.5 101.8) (width 0.3) (layer "F.Cu") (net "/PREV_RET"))
 (segment (start 103 101.85) (end 103 101.8) (width 0.3) (layer "F.Cu") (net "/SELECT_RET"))
 (segment (start 104.4 102) (end 104.3 101.9) (width 0.3) (layer "F.Cu") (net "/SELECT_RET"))
 (segment (start 103 101.85) (end 103 101.8) (width 0.3) (layer "F.Cu") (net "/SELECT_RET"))
 (segment (start 105.2 102) (end 104.4 102) (width 0.3) (layer "F.Cu") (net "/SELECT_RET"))
 (segment (start 103.6 101.8) (end 103 101.8) (width 0.3) (layer "F.Cu") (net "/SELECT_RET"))
 (segment (start 97 101.85) (end 97 101.8) (width 0.3) (layer "F.Cu") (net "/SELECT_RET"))
 (segment (start 97 101.85) (end 97 101.8) (width 0.3) (layer "F.Cu") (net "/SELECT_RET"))
 (segment (start 103 101.85) (end 103 101.8) (width 0.3) (layer "F.Cu") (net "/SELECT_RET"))
 (segment (start 97 101.8) (end 103 101.8) (width 0.3) (layer "F.Cu") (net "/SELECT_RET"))
 (segment (start 105.175 102) (end 105.2 102) (width 0.3) (layer "F.Cu") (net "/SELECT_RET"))
 (segment (start 103.7 101.9) (end 103.6 101.8) (width 0.3) (layer "F.Cu") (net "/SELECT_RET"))
 (segment (start 103 101.85) (end 103 101.8) (width 0.3) (layer "F.Cu") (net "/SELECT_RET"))
 (segment (start 104.3 101.9) (end 103.7 101.9) (width 0.3) (layer "F.Cu") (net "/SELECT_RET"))
 (segment (start 97.46 108.46) (end 97.5 108.5) (width 0.3) (layer "F.Cu") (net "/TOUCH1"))
 (segment (start 96.3 107.3) (end 96.3 106.8) (width 0.3) (layer "F.Cu") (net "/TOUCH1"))
 (segment (start 96.3 106.8) (end 95.5 106) (width 0.3) (layer "F.Cu") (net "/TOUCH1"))
 (segment (start 97.5 108.5) (end 96.3 107.3) (width 0.3) (layer "F.Cu") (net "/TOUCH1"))
 (segment (start 100 111) (end 100 113) (width 0.3) (layer "F.Cu") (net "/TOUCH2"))
 (segment (start 100 108.5) (end 100 106) (width 0.3) (layer "F.Cu") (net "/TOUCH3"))
 (segment (start 100 108.46) (end 100 108.5) (width 0.3) (layer "F.Cu") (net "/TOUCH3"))
 (segment (start 102.5 111) (end 102.5 113) (width 0.3) (layer "F.Cu") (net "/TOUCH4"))
 (segment (start 102.54 113) (end 102.5 113) (width 0.3) (layer "F.Cu") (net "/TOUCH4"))
 (segment (start 102.54 113) (end 102.5 113) (width 0.3) (layer "F.Cu") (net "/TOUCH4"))
 (segment (start 102.54 111) (end 102.5 111) (width 0.3) (layer "F.Cu") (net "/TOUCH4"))
 (segment (start 102.54 108.46) (end 102.5 108.5) (width 0.3) (layer "F.Cu") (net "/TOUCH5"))
 (segment (start 102.5 108.5) (end 103.7 107.3) (width 0.3) (layer "F.Cu") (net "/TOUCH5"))
 (segment (start 103.7 106.8) (end 104.5 106) (width 0.3) (layer "F.Cu") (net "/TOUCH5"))
 (segment (start 103.7 107.3) (end 103.7 106.8) (width 0.3) (layer "F.Cu") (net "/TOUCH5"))
 (segment (start 105.08 113) (end 105.1 113) (width 0.3) (layer "F.Cu") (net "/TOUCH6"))
 (segment (start 105.08 111) (end 105.1 111) (width 0.3) (layer "F.Cu") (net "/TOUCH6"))
 (segment (start 105.08 113) (end 105.1 113) (width 0.3) (layer "F.Cu") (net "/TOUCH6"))
 (segment (start 105.1 111) (end 105.1 113) (width 0.3) (layer "F.Cu") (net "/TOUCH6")))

